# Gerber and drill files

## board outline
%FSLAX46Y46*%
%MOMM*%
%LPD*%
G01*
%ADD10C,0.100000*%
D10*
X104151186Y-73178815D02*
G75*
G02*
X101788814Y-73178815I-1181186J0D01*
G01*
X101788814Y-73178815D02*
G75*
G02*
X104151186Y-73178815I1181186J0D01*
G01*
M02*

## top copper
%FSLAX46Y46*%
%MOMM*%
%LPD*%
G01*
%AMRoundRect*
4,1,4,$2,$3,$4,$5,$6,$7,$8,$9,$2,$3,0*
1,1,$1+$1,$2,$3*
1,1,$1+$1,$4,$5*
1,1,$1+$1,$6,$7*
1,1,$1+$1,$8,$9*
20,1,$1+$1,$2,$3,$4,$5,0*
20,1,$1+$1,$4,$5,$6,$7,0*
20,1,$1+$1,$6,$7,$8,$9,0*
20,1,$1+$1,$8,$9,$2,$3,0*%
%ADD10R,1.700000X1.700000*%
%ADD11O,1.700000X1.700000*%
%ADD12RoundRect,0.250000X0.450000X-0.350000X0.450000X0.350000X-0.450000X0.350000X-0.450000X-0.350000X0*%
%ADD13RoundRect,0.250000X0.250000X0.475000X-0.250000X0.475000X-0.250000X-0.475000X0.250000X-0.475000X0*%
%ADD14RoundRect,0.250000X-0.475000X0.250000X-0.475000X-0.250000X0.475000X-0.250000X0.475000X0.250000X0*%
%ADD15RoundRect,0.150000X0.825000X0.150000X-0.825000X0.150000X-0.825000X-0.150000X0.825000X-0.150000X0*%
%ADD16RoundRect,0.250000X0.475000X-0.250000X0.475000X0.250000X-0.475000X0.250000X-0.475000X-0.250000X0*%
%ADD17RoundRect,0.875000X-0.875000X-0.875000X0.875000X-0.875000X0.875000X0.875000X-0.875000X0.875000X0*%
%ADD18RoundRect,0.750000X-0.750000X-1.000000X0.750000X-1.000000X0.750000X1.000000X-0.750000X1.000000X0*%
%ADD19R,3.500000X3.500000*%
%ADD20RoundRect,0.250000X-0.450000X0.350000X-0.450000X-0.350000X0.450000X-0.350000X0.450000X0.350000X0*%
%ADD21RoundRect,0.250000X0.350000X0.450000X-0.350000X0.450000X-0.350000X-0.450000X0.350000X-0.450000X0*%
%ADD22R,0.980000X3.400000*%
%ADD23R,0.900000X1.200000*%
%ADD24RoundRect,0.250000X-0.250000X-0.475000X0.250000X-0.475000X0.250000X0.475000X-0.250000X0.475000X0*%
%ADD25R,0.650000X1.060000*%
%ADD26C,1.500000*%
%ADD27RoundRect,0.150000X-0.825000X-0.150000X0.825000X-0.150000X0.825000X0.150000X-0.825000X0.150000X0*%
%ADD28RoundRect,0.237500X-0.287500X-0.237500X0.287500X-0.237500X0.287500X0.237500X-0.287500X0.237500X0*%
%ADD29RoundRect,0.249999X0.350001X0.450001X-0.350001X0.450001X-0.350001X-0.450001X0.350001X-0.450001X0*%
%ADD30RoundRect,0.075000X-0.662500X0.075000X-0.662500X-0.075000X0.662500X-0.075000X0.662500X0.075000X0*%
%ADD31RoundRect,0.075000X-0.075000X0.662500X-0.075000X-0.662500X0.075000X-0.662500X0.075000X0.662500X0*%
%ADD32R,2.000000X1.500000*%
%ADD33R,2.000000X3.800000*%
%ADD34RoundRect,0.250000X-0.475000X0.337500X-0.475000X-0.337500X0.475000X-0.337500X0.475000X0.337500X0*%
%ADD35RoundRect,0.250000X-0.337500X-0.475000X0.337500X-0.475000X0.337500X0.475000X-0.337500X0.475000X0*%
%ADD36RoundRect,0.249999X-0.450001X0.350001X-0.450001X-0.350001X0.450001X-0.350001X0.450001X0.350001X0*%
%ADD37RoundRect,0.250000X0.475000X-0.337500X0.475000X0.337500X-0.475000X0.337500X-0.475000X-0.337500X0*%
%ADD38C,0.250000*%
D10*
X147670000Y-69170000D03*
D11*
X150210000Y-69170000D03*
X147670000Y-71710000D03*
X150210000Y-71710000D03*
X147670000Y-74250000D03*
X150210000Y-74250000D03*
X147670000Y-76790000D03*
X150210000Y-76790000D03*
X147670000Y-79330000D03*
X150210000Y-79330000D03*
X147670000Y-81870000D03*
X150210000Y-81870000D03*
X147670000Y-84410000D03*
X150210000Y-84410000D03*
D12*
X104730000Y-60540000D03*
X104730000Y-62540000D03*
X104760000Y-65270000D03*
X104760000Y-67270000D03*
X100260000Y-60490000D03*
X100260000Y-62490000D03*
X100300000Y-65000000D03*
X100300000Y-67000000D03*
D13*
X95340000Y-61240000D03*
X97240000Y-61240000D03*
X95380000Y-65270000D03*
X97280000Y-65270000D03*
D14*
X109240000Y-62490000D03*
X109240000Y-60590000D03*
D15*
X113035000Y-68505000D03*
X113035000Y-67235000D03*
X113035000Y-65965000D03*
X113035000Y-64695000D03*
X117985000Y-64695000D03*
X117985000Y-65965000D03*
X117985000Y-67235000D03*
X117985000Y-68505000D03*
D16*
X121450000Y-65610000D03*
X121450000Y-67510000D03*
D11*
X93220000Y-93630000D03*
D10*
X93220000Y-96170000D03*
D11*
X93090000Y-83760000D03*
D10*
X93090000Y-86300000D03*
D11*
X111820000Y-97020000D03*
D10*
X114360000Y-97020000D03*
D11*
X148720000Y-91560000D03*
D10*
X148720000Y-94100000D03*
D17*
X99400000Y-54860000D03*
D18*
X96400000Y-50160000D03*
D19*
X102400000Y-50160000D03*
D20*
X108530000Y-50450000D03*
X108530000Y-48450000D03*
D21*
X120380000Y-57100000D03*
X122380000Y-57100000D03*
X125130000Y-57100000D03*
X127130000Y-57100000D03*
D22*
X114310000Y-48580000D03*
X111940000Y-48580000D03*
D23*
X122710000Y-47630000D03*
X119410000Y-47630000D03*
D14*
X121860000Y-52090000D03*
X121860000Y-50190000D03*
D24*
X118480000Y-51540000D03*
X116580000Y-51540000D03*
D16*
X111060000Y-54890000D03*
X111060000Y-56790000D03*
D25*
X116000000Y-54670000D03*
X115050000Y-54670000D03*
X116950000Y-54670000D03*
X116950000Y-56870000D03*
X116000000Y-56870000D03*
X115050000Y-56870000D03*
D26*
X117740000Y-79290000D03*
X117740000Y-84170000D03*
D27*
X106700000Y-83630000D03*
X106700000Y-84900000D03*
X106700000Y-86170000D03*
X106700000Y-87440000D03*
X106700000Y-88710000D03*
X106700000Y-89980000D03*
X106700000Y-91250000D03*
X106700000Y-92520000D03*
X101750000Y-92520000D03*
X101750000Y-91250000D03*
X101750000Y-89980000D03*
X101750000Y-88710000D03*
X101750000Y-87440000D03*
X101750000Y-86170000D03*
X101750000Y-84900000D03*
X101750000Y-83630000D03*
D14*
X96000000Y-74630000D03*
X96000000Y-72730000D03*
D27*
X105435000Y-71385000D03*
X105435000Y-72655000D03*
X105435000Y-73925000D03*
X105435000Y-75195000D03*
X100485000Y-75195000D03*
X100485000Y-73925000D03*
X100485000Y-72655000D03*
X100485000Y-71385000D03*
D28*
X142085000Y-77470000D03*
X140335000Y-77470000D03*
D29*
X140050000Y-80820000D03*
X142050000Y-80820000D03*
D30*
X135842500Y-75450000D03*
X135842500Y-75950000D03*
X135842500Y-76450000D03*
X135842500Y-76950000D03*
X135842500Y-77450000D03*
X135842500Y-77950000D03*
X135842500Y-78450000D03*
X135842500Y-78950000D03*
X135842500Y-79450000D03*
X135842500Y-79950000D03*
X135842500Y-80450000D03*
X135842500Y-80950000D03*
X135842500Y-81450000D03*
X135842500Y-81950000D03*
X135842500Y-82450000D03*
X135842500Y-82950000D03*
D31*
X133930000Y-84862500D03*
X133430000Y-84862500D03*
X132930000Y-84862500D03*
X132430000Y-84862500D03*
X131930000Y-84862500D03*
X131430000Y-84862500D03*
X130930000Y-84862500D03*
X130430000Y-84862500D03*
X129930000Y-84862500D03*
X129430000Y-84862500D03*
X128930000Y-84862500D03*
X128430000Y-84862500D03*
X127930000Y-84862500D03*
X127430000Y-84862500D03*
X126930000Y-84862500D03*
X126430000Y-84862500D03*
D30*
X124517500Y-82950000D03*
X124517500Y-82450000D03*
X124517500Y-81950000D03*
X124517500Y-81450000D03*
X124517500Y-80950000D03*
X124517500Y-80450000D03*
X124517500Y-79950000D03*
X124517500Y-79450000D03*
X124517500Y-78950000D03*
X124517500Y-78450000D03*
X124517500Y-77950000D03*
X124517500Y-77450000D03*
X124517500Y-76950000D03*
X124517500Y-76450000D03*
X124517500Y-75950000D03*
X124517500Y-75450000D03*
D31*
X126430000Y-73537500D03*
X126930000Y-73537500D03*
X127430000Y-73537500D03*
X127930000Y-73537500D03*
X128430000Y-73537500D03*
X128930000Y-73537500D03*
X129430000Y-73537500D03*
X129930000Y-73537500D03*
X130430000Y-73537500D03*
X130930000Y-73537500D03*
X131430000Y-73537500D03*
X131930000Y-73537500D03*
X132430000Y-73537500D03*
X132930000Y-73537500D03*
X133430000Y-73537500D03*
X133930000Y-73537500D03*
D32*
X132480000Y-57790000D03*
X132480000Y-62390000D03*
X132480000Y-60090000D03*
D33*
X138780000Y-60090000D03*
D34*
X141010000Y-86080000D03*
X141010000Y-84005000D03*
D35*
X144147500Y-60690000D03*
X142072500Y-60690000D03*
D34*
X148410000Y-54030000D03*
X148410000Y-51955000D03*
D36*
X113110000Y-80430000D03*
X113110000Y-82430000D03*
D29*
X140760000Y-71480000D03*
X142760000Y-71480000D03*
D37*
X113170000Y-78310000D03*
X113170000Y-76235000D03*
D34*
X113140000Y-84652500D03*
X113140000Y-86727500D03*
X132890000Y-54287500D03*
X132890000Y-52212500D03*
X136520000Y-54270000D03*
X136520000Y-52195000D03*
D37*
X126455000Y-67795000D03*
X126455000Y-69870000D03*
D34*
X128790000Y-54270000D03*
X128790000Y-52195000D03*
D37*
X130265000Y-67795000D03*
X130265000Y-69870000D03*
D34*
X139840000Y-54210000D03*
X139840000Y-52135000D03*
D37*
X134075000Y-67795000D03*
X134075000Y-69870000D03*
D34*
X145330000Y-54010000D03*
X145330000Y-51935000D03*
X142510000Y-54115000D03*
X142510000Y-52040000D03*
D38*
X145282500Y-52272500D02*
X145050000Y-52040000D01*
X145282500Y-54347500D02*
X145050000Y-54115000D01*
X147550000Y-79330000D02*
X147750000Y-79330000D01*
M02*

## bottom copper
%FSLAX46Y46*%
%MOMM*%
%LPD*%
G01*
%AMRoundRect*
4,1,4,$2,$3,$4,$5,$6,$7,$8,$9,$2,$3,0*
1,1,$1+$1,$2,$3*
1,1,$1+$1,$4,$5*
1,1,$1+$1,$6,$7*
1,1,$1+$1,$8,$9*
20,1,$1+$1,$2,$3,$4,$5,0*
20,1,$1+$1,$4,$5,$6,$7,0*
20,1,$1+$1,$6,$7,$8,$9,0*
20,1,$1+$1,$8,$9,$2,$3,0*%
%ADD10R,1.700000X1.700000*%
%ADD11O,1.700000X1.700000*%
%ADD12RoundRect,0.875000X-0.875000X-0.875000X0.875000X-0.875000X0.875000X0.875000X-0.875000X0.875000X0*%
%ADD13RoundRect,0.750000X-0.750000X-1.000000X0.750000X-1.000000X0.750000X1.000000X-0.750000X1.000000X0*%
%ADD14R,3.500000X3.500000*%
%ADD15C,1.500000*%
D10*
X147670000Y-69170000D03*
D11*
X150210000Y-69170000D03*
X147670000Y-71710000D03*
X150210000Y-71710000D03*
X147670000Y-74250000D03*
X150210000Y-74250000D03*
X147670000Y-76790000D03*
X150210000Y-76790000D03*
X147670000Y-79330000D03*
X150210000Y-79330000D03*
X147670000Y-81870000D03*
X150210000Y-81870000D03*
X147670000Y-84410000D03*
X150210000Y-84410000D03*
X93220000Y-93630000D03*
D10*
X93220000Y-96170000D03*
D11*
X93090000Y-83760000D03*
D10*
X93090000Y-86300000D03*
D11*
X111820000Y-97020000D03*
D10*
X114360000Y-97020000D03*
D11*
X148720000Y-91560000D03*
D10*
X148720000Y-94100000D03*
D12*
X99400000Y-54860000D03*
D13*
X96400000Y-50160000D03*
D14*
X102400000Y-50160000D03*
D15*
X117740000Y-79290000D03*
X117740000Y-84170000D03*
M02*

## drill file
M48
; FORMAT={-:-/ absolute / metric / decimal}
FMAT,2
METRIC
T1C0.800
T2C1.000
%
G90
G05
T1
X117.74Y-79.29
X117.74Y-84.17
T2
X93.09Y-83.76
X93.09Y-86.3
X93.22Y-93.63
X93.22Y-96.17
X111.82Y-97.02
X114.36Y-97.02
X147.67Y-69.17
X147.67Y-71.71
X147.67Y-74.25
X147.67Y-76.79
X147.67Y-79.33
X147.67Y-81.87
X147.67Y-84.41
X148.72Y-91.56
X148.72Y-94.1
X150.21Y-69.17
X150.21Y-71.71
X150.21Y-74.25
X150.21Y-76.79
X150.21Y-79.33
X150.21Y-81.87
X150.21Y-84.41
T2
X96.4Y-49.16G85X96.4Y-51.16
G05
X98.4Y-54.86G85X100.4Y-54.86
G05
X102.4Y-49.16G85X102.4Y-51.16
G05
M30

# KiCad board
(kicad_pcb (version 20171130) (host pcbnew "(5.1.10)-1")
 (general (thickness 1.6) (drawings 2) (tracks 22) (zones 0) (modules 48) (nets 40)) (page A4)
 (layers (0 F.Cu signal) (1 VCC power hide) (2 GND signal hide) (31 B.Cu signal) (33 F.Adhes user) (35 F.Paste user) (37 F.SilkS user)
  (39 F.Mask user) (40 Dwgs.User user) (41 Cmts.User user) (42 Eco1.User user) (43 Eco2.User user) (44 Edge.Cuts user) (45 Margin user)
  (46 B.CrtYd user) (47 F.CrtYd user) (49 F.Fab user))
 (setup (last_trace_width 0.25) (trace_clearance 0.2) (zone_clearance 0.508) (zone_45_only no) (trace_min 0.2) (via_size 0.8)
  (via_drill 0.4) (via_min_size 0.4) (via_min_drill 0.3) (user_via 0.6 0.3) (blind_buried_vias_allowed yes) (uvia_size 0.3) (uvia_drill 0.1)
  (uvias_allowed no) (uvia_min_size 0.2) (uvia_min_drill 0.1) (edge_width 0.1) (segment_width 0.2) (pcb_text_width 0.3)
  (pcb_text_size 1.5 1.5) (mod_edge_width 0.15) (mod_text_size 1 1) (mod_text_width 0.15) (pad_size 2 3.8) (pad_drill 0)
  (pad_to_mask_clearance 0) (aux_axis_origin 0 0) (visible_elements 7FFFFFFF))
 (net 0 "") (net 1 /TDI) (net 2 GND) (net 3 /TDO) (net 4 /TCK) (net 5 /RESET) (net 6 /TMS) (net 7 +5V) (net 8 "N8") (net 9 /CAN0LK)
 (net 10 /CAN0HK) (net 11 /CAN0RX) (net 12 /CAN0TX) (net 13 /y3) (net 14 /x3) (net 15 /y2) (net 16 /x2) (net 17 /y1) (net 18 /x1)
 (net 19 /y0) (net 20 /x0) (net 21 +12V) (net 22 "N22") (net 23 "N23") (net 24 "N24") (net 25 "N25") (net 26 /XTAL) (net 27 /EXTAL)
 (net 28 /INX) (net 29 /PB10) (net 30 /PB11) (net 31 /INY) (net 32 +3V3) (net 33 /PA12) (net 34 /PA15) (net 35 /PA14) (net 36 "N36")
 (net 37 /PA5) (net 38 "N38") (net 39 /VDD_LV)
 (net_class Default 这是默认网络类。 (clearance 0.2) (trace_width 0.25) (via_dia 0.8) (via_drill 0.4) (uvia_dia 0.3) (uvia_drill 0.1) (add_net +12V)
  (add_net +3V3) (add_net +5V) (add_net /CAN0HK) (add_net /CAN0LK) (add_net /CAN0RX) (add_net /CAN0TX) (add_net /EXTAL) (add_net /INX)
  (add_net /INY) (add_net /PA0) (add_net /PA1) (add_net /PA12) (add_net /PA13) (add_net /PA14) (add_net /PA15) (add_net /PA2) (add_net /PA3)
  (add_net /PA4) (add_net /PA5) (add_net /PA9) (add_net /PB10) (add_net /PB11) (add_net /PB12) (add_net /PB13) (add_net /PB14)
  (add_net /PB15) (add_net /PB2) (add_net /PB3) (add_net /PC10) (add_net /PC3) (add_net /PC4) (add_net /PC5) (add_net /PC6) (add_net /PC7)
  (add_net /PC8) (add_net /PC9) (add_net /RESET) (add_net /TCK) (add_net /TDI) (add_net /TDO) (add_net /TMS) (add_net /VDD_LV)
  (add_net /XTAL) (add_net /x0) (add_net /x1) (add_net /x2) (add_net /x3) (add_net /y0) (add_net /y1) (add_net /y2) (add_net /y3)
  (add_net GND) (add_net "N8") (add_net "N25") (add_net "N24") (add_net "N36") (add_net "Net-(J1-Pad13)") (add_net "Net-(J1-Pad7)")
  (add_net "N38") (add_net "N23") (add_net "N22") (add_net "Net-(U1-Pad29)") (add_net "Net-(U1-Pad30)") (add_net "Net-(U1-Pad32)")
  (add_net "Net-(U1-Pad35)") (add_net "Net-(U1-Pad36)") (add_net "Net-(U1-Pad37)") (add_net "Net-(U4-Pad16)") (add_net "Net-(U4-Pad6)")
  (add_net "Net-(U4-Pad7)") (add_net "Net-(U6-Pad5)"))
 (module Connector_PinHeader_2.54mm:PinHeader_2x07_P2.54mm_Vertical (layer F.Cu) (at 147.67 69.17)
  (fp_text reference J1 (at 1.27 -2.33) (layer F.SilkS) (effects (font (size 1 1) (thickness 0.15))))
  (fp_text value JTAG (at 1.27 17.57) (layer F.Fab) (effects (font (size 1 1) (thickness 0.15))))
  (pad 1 thru_hole rect (at 0 0) (size 1.7 1.7) (drill 1) (layers *.Cu *.Mask) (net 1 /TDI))
  (pad 2 thru_hole oval (at 2.54 0) (size 1.7 1.7) (drill 1) (layers *.Cu *.Mask) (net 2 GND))
  (pad 3 thru_hole oval (at 0 2.54) (size 1.7 1.7) (drill 1) (layers *.Cu *.Mask) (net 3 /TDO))
  (pad 4 thru_hole oval (at 2.54 2.54) (size 1.7 1.7) (drill 1) (layers *.Cu *.Mask) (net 2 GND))
  (pad 5 thru_hole oval (at 0 5.08) (size 1.7 1.7) (drill 1) (layers *.Cu *.Mask) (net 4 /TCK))
  (pad 6 thru_hole oval (at 2.54 5.08) (size 1.7 1.7) (drill 1) (layers *.Cu *.Mask) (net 2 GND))
  (pad 7 thru_hole oval (at 0 7.62) (size 1.7 1.7) (drill 1) (layers *.Cu *.Mask))
  (pad 8 thru_hole oval (at 2.54 7.62) (size 1.7 1.7) (drill 1) (layers *.Cu *.Mask) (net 2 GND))
  (pad 9 thru_hole oval (at 0 10.16) (size 1.7 1.7) (drill 1) (layers *.Cu *.Mask) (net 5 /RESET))
  (pad 10 thru_hole oval (at 2.54 10.16) (size 1.7 1.7) (drill 1) (layers *.Cu *.Mask) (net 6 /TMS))
  (pad 11 thru_hole oval (at 0 12.7) (size 1.7 1.7) (drill 1) (layers *.Cu *.Mask) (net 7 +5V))
  (pad 12 thru_hole oval (at 2.54 12.7) (size 1.7 1.7) (drill 1) (layers *.Cu *.Mask) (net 2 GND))
  (pad 13 thru_hole oval (at 0 15.24) (size 1.7 1.7) (drill 1) (layers *.Cu *.Mask))
  (pad 14 thru_hole oval (at 2.54 15.24) (size 1.7 1.7) (drill 1) (layers *.Cu *.Mask) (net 2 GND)))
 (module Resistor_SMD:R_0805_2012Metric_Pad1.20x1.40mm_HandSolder (layer F.Cu) (at 104.73 61.54 90)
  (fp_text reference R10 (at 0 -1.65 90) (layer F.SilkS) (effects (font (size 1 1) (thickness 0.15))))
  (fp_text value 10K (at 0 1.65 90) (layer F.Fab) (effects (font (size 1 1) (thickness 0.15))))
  (pad 2 smd roundrect (at 1 0 90) (size 1.2 1.4) (layers F.Cu F.Paste F.Mask) (roundrect_rratio 0.208333) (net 2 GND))
  (pad 1 smd roundrect (at -1 0 90) (size 1.2 1.4) (layers F.Cu F.Paste F.Mask) (roundrect_rratio 0.208333) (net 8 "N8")))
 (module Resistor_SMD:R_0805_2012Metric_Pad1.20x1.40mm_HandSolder (layer F.Cu) (at 104.76 66.27 90)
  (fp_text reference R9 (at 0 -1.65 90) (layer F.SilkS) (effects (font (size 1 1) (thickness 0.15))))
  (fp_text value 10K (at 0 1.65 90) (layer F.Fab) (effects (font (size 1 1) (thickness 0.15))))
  (pad 2 smd roundrect (at 1 0 90) (size 1.2 1.4) (layers F.Cu F.Paste F.Mask) (roundrect_rratio 0.208333) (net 8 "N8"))
  (pad 1 smd roundrect (at -1 0 90) (size 1.2 1.4) (layers F.Cu F.Paste F.Mask) (roundrect_rratio 0.208333) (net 7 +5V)))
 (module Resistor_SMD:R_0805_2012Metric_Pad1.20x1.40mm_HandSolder (layer F.Cu) (at 100.26 61.49 90)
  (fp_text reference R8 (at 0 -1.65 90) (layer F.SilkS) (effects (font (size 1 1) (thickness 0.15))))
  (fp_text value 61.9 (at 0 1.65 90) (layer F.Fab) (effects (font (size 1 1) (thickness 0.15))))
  (pad 2 smd roundrect (at 1 0 90) (size 1.2 1.4) (layers F.Cu F.Paste F.Mask) (roundrect_rratio 0.208333) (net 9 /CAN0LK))
  (pad 1 smd roundrect (at -1 0 90) (size 1.2 1.4) (layers F.Cu F.Paste F.Mask) (roundrect_rratio 0.208333) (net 8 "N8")))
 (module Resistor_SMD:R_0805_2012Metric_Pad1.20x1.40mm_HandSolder (layer F.Cu) (at 100.3 66 90)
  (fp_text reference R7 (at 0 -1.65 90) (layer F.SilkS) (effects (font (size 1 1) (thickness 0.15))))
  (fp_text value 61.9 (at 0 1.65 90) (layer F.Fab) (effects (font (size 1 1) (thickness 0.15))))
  (pad 2 smd roundrect (at 1 0 90) (size 1.2 1.4) (layers F.Cu F.Paste F.Mask) (roundrect_rratio 0.208333) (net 8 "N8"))
  (pad 1 smd roundrect (at -1 0 90) (size 1.2 1.4) (layers F.Cu F.Paste F.Mask) (roundrect_rratio 0.208333) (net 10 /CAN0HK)))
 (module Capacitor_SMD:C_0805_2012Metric (layer F.Cu) (at 96.29 61.24 180)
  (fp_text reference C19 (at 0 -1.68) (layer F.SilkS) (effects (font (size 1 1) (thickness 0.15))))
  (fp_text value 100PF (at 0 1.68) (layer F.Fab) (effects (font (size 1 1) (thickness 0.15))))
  (pad 2 smd roundrect (at 0.95 0 180) (size 1 1.45) (layers F.Cu F.Paste F.Mask) (roundrect_rratio 0.25) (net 2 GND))
  (pad 1 smd roundrect (at -0.95 0 180) (size 1 1.45) (layers F.Cu F.Paste F.Mask) (roundrect_rratio 0.25) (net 9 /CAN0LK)))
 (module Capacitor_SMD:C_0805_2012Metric (layer F.Cu) (at 96.33 65.27 180)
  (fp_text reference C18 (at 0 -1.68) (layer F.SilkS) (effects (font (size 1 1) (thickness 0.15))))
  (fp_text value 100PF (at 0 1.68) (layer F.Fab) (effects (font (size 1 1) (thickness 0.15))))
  (pad 2 smd roundrect (at 0.95 0 180) (size 1 1.45) (layers F.Cu F.Paste F.Mask) (roundrect_rratio 0.25) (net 2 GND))
  (pad 1 smd roundrect (at -0.95 0 180) (size 1 1.45) (layers F.Cu F.Paste F.Mask) (roundrect_rratio 0.25) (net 10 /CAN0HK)))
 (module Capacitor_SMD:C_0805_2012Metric (layer F.Cu) (at 109.24 61.54 270)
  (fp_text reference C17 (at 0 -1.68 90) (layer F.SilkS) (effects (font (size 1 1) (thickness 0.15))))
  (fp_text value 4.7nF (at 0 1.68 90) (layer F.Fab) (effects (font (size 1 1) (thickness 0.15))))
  (pad 2 smd roundrect (at 0.95 0 270) (size 1 1.45) (layers F.Cu F.Paste F.Mask) (roundrect_rratio 0.25) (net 8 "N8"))
  (pad 1 smd roundrect (at -0.95 0 270) (size 1 1.45) (layers F.Cu F.Paste F.Mask) (roundrect_rratio 0.25) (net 2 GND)))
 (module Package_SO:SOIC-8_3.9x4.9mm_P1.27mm (layer F.Cu) (at 115.51 66.6 180)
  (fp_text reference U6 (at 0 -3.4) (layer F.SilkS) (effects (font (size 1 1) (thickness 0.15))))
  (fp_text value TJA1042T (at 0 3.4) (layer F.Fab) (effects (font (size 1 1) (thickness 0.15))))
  (pad 8 smd roundrect (at 2.475 -1.905 180) (size 1.95 0.6) (layers F.Cu F.Paste F.Mask) (roundrect_rratio 0.25) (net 2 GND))
  (pad 7 smd roundrect (at 2.475 -0.635 180) (size 1.95 0.6) (layers F.Cu F.Paste F.Mask) (roundrect_rratio 0.25) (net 10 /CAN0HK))
  (pad 6 smd roundrect (at 2.475 0.635 180) (size 1.95 0.6) (layers F.Cu F.Paste F.Mask) (roundrect_rratio 0.25) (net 9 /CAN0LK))
  (pad 5 smd roundrect (at 2.475 1.905 180) (size 1.95 0.6) (layers F.Cu F.Paste F.Mask) (roundrect_rratio 0.25))
  (pad 4 smd roundrect (at -2.475 1.905 180) (size 1.95 0.6) (layers F.Cu F.Paste F.Mask) (roundrect_rratio 0.25) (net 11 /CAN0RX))
  (pad 3 smd roundrect (at -2.475 0.635 180) (size 1.95 0.6) (layers F.Cu F.Paste F.Mask) (roundrect_rratio 0.25) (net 7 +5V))
  (pad 2 smd roundrect (at -2.475 -0.635 180) (size 1.95 0.6) (layers F.Cu F.Paste F.Mask) (roundrect_rratio 0.25) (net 2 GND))
  (pad 1 smd roundrect (at -2.475 -1.905 180) (size 1.95 0.6) (layers F.Cu F.Paste F.Mask) (roundrect_rratio 0.25) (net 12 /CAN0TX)))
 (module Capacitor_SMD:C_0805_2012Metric (layer F.Cu) (at 121.45 66.56 90)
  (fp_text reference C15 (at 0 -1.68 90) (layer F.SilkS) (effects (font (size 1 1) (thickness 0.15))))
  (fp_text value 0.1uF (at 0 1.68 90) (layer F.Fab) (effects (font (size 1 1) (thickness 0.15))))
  (pad 2 smd roundrect (at 0.95 0 90) (size 1 1.45) (layers F.Cu F.Paste F.Mask) (roundrect_rratio 0.25) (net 7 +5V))
  (pad 1 smd roundrect (at -0.95 0 90) (size 1 1.45) (layers F.Cu F.Paste F.Mask) (roundrect_rratio 0.25) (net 2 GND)))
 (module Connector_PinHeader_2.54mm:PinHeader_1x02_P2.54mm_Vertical (layer F.Cu) (at 93.22 96.17 180)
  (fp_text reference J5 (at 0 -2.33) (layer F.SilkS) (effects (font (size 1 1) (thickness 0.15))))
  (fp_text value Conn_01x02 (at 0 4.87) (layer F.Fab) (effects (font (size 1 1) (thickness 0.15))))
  (pad 2 thru_hole oval (at 0 2.54 180) (size 1.7 1.7) (drill 1) (layers *.Cu *.Mask) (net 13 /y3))
  (pad 1 thru_hole rect (at 0 0 180) (size 1.7 1.7) (drill 1) (layers *.Cu *.Mask) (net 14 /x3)))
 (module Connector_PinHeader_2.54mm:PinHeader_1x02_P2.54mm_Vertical (layer F.Cu) (at 93.09 86.3 180)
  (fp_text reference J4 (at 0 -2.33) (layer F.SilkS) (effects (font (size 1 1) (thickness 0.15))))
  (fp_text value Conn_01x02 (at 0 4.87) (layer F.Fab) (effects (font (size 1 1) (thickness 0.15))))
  (pad 2 thru_hole oval (at 0 2.54 180) (size 1.7 1.7) (drill 1) (layers *.Cu *.Mask) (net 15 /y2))
  (pad 1 thru_hole rect (at 0 0 180) (size 1.7 1.7) (drill 1) (layers *.Cu *.Mask) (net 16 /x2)))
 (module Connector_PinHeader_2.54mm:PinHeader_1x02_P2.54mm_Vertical (layer F.Cu) (at 114.36 97.02 270)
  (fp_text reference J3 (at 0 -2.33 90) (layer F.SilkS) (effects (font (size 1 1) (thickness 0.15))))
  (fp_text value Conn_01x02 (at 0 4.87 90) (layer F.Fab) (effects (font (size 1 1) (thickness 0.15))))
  (pad 2 thru_hole oval (at 0 2.54 270) (size 1.7 1.7) (drill 1) (layers *.Cu *.Mask) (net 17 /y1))
  (pad 1 thru_hole rect (at 0 0 270) (size 1.7 1.7) (drill 1) (layers *.Cu *.Mask) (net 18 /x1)))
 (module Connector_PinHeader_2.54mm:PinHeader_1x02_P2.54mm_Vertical (layer F.Cu) (at 148.72 94.1 180)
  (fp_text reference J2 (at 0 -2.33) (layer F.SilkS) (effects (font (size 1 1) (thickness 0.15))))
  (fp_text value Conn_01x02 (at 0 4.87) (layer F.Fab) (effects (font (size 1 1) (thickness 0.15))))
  (pad 2 thru_hole oval (at 0 2.54 180) (size 1.7 1.7) (drill 1) (layers *.Cu *.Mask) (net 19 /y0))
  (pad 1 thru_hole rect (at 0 0 180) (size 1.7 1.7) (drill 1) (layers *.Cu *.Mask) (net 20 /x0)))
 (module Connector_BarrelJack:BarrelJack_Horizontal (layer F.Cu) (at 102.4 50.16)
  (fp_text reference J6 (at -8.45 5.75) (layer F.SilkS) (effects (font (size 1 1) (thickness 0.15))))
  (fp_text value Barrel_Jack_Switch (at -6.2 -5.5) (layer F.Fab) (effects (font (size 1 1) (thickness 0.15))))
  (pad 3 thru_hole roundrect (at -3 4.7) (size 3.5 3.5) (drill oval 3 1) (layers *.Cu *.Mask) (roundrect_rratio 0.25) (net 2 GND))
  (pad 2 thru_hole roundrect (at -6 0) (size 3 3.5) (drill oval 1 3) (layers *.Cu *.Mask) (roundrect_rratio 0.25) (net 2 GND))
  (pad 1 thru_hole rect (at 0 0) (size 3.5 3.5) (drill oval 1 3) (layers *.Cu *.Mask) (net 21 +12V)))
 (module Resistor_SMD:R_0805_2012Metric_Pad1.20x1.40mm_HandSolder (layer F.Cu) (at 108.53 49.45 270)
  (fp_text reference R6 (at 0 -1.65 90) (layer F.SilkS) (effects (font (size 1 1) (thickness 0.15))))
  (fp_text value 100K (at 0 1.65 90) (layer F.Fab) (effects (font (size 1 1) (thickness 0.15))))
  (pad 2 smd roundrect (at 1 0 270) (size 1.2 1.4) (layers F.Cu F.Paste F.Mask) (roundrect_rratio 0.208333) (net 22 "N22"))
  (pad 1 smd roundrect (at -1 0 270) (size 1.2 1.4) (layers F.Cu F.Paste F.Mask) (roundrect_rratio 0.208333) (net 21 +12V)))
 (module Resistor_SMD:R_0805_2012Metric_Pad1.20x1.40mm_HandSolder (layer F.Cu) (at 121.38 57.1 180)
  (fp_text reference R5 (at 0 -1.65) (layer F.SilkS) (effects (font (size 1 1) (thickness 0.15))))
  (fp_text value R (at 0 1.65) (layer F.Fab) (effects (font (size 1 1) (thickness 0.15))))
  (pad 2 smd roundrect (at 1 0 180) (size 1.2 1.4) (layers F.Cu F.Paste F.Mask) (roundrect_rratio 0.208333) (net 2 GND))
  (pad 1 smd roundrect (at -1 0 180) (size 1.2 1.4) (layers F.Cu F.Paste F.Mask) (roundrect_rratio 0.208333) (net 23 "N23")))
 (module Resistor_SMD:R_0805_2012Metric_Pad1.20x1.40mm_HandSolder (layer F.Cu) (at 126.13 57.1 180)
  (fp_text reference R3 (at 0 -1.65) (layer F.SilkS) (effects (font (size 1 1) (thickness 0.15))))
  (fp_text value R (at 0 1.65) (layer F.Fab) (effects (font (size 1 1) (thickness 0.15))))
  (pad 2 smd roundrect (at 1 0 180) (size 1.2 1.4) (layers F.Cu F.Paste F.Mask) (roundrect_rratio 0.208333) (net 23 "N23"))
  (pad 1 smd roundrect (at -1 0 180) (size 1.2 1.4) (layers F.Cu F.Paste F.Mask) (roundrect_rratio 0.208333) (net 7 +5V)))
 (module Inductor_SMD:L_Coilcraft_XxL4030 (layer F.Cu) (at 113.125 48.58)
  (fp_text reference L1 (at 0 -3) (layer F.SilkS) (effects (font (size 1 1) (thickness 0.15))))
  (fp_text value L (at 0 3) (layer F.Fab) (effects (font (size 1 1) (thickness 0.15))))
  (pad 2 smd rect (at 1.185 0) (size 0.98 3.4) (layers F.Cu F.Paste F.Mask) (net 7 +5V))
  (pad 1 smd rect (at -1.185 0) (size 0.98 3.4) (layers F.Cu F.Paste F.Mask) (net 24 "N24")))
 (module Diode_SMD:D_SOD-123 (layer F.Cu) (at 121.06 47.63)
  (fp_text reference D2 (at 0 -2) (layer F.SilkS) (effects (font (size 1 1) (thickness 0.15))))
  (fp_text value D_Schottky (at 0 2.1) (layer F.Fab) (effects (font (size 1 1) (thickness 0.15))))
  (pad 2 smd rect (at 1.65 0) (size 0.9 1.2) (layers F.Cu F.Paste F.Mask) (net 2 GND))
  (pad 1 smd rect (at -1.65 0) (size 0.9 1.2) (layers F.Cu F.Paste F.Mask) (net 24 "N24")))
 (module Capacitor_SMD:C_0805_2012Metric (layer F.Cu) (at 121.86 51.14 270)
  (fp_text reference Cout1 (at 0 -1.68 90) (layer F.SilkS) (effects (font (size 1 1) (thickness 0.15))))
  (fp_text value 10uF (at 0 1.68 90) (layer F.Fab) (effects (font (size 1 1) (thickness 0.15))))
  (pad 2 smd roundrect (at 0.95 0 270) (size 1 1.45) (layers F.Cu F.Paste F.Mask) (roundrect_rratio 0.25) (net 2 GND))
  (pad 1 smd roundrect (at -0.95 0 270) (size 1 1.45) (layers F.Cu F.Paste F.Mask) (roundrect_rratio 0.25) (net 7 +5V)))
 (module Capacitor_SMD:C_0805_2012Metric (layer F.Cu) (at 117.53 51.54)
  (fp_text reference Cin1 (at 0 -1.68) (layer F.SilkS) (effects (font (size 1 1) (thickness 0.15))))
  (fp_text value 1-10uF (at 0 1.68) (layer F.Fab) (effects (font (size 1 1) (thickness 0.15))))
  (pad 2 smd roundrect (at 0.95 0) (size 1 1.45) (layers F.Cu F.Paste F.Mask) (roundrect_rratio 0.25) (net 2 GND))
  (pad 1 smd roundrect (at -0.95 0) (size 1 1.45) (layers F.Cu F.Paste F.Mask) (roundrect_rratio 0.25) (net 21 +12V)))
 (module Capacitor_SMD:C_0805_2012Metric (layer F.Cu) (at 111.06 55.84 90)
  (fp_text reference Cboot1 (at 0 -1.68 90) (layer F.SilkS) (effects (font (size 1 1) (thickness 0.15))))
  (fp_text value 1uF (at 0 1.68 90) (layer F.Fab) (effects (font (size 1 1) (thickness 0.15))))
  (pad 2 smd roundrect (at 0.95 0 90) (size 1 1.45) (layers F.Cu F.Paste F.Mask) (roundrect_rratio 0.25) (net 24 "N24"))
  (pad 1 smd roundrect (at -0.95 0 90) (size 1 1.45) (layers F.Cu F.Paste F.Mask) (roundrect_rratio 0.25) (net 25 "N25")))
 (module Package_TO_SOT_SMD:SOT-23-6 (layer F.Cu) (at 116 55.77 90)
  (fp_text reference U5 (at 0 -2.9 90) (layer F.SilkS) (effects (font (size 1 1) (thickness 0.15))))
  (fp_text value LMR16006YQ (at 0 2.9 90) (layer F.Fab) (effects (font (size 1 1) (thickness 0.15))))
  (pad 5 smd rect (at 1.1 0 90) (size 1.06 0.65) (layers F.Cu F.Paste F.Mask) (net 21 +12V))
  (pad 6 smd rect (at 1.1 -0.95 90) (size 1.06 0.65) (layers F.Cu F.Paste F.Mask) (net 24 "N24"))
  (pad 4 smd rect (at 1.1 0.95 90) (size 1.06 0.65) (layers F.Cu F.Paste F.Mask) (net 22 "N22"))
  (pad 3 smd rect (at -1.1 0.95 90) (size 1.06 0.65) (layers F.Cu F.Paste F.Mask) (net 23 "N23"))
  (pad 2 smd rect (at -1.1 0 90) (size 1.06 0.65) (layers F.Cu F.Paste F.Mask) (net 2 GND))
  (pad 1 smd rect (at -1.1 -0.95 90) (size 1.06 0.65) (layers F.Cu F.Paste F.Mask) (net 25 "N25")))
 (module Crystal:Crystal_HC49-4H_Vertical (layer F.Cu) (at 117.74 84.17 90)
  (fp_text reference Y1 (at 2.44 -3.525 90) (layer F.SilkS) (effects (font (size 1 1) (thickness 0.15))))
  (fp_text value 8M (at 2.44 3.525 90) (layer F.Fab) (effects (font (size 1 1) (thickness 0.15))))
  (pad 2 thru_hole circle (at 4.88 0 90) (size 1.5 1.5) (drill 0.8) (layers *.Cu *.Mask) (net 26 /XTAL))
  (pad 1 thru_hole circle (at 0 0 90) (size 1.5 1.5) (drill 0.8) (layers *.Cu *.Mask) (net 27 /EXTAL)))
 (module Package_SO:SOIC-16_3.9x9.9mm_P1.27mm (layer F.Cu) (at 104.225 88.075)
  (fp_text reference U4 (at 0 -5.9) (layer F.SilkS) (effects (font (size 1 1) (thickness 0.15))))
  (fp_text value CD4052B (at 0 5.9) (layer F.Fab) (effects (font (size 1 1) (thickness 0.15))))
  (pad 16 smd roundrect (at 2.475 -4.445) (size 1.95 0.6) (layers F.Cu F.Paste F.Mask) (roundrect_rratio 0.25))
  (pad 15 smd roundrect (at 2.475 -3.175) (size 1.95 0.6) (layers F.Cu F.Paste F.Mask) (roundrect_rratio 0.25) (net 16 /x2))
  (pad 14 smd roundrect (at 2.475 -1.905) (size 1.95 0.6) (layers F.Cu F.Paste F.Mask) (roundrect_rratio 0.25) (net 18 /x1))
  (pad 13 smd roundrect (at 2.475 -0.635) (size 1.95 0.6) (layers F.Cu F.Paste F.Mask) (roundrect_rratio 0.25) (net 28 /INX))
  (pad 12 smd roundrect (at 2.475 0.635) (size 1.95 0.6) (layers F.Cu F.Paste F.Mask) (roundrect_rratio 0.25) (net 20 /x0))
  (pad 11 smd roundrect (at 2.475 1.905) (size 1.95 0.6) (layers F.Cu F.Paste F.Mask) (roundrect_rratio 0.25) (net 14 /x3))
  (pad 10 smd roundrect (at 2.475 3.175) (size 1.95 0.6) (layers F.Cu F.Paste F.Mask) (roundrect_rratio 0.25) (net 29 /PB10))
  (pad 9 smd roundrect (at 2.475 4.445) (size 1.95 0.6) (layers F.Cu F.Paste F.Mask) (roundrect_rratio 0.25) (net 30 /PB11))
  (pad 8 smd roundrect (at -2.475 4.445) (size 1.95 0.6) (layers F.Cu F.Paste F.Mask) (roundrect_rratio 0.25) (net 2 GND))
  (pad 7 smd roundrect (at -2.475 3.175) (size 1.95 0.6) (layers F.Cu F.Paste F.Mask) (roundrect_rratio 0.25))
  (pad 6 smd roundrect (at -2.475 1.905) (size 1.95 0.6) (layers F.Cu F.Paste F.Mask) (roundrect_rratio 0.25))
  (pad 5 smd roundrect (at -2.475 0.635) (size 1.95 0.6) (layers F.Cu F.Paste F.Mask) (roundrect_rratio 0.25) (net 17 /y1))
  (pad 4 smd roundrect (at -2.475 -0.635) (size 1.95 0.6) (layers F.Cu F.Paste F.Mask) (roundrect_rratio 0.25) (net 13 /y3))
  (pad 3 smd roundrect (at -2.475 -1.905) (size 1.95 0.6) (layers F.Cu F.Paste F.Mask) (roundrect_rratio 0.25) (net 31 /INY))
  (pad 2 smd roundrect (at -2.475 -3.175) (size 1.95 0.6) (layers F.Cu F.Paste F.Mask) (roundrect_rratio 0.25) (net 15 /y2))
  (pad 1 smd roundrect (at -2.475 -4.445) (size 1.95 0.6) (layers F.Cu F.Paste F.Mask) (roundrect_rratio 0.25) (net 19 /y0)))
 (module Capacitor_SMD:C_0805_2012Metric (layer F.Cu) (at 96 73.68 270)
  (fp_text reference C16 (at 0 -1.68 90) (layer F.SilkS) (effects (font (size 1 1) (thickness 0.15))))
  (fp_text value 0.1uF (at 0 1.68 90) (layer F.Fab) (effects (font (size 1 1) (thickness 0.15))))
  (pad 2 smd roundrect (at 0.95 0 270) (size 1 1.45) (layers F.Cu F.Paste F.Mask) (roundrect_rratio 0.25) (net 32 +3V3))
  (pad 1 smd roundrect (at -0.95 0 270) (size 1 1.45) (layers F.Cu F.Paste F.Mask) (roundrect_rratio 0.25) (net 2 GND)))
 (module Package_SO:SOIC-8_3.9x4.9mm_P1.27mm (layer F.Cu) (at 102.96 73.29)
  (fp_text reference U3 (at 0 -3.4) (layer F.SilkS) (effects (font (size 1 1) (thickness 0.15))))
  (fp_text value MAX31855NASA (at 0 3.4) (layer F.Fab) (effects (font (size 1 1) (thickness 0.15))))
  (pad 8 smd roundrect (at 2.475 -1.905) (size 1.95 0.6) (layers F.Cu F.Paste F.Mask) (roundrect_rratio 0.25))
  (pad 7 smd roundrect (at 2.475 -0.635) (size 1.95 0.6) (layers F.Cu F.Paste F.Mask) (roundrect_rratio 0.25) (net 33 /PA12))
  (pad 6 smd roundrect (at 2.475 0.635) (size 1.95 0.6) (layers F.Cu F.Paste F.Mask) (roundrect_rratio 0.25) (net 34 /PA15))
  (pad 5 smd roundrect (at 2.475 1.905) (size 1.95 0.6) (layers F.Cu F.Paste F.Mask) (roundrect_rratio 0.25) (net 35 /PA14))
  (pad 4 smd roundrect (at -2.475 1.905) (size 1.95 0.6) (layers F.Cu F.Paste F.Mask) (roundrect_rratio 0.25) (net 32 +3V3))
  (pad 3 smd roundrect (at -2.475 0.635) (size 1.95 0.6) (layers F.Cu F.Paste F.Mask) (roundrect_rratio 0.25) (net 28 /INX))
  (pad 2 smd roundrect (at -2.475 -0.635) (size 1.95 0.6) (layers F.Cu F.Paste F.Mask) (roundrect_rratio 0.25) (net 31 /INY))
  (pad 1 smd roundrect (at -2.475 -1.905) (size 1.95 0.6) (layers F.Cu F.Paste F.Mask) (roundrect_rratio 0.25) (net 2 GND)))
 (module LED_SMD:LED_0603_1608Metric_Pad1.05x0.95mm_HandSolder (layer F.Cu) (at 141.21 77.47)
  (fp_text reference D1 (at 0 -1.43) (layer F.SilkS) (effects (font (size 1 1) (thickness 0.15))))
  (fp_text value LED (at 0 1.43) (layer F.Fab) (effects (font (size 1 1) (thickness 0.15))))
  (pad 2 smd roundrect (at 0.875 0) (size 1.05 0.95) (layers F.Cu F.Paste F.Mask) (roundrect_rratio 0.25) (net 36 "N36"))
  (pad 1 smd roundrect (at -0.875 0) (size 1.05 0.95) (layers F.Cu F.Paste F.Mask) (roundrect_rratio 0.25) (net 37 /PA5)))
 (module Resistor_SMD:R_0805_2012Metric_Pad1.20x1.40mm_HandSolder (layer F.Cu) (at 141.05 80.82 180)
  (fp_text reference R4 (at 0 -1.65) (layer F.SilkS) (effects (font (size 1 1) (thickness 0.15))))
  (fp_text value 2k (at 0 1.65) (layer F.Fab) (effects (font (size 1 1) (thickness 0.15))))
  (pad 2 smd roundrect (at 1 0 180) (size 1.2 1.4) (layers F.Cu F.Paste F.Mask) (roundrect_rratio 0.2083325) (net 7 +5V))
  (pad 1 smd roundrect (at -1 0 180) (size 1.2 1.4) (layers F.Cu F.Paste F.Mask) (roundrect_rratio 0.2083325) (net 36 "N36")))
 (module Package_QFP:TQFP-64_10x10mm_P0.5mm (layer F.Cu) (at 130.18 79.2 270)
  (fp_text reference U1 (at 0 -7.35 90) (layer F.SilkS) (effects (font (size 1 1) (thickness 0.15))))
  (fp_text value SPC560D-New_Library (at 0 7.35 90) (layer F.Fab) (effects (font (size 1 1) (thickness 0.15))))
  (pad 64 smd roundrect (at -3.75 -5.6625 270) (size 0.3 1.475) (layers F.Cu F.Paste F.Mask) (roundrect_rratio 0.25))
  (pad 63 smd roundrect (at -3.25 -5.6625 270) (size 0.3 1.475) (layers F.Cu F.Paste F.Mask) (roundrect_rratio 0.25))
  (pad 62 smd roundrect (at -2.75 -5.6625 270) (size 0.3 1.475) (layers F.Cu F.Paste F.Mask) (roundrect_rratio 0.25))
  (pad 61 smd roundrect (at -2.25 -5.6625 270) (size 0.3 1.475) (layers F.Cu F.Paste F.Mask) (roundrect_rratio 0.25))
  (pad 60 smd roundrect (at -1.75 -5.6625 270) (size 0.3 1.475) (layers F.Cu F.Paste F.Mask) (roundrect_rratio 0.25) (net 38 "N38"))
  (pad 59 smd roundrect (at -1.25 -5.6625 270) (size 0.3 1.475) (layers F.Cu F.Paste F.Mask) (roundrect_rratio 0.25) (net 1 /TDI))
  (pad 58 smd roundrect (at -0.75 -5.6625 270) (size 0.3 1.475) (layers F.Cu F.Paste F.Mask) (roundrect_rratio 0.25) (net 2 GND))
  (pad 57 smd roundrect (at -0.25 -5.6625 270) (size 0.3 1.475) (layers F.Cu F.Paste F.Mask) (roundrect_rratio 0.25) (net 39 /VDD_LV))
  (pad 56 smd roundrect (at 0.25 -5.6625 270) (size 0.3 1.475) (layers F.Cu F.Paste F.Mask) (roundrect_rratio 0.25) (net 7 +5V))
  (pad 55 smd roundrect (at 0.75 -5.6625 270) (size 0.3 1.475) (layers F.Cu F.Paste F.Mask) (roundrect_rratio 0.25) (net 2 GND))
  (pad 54 smd roundrect (at 1.25 -5.6625 270) (size 0.3 1.475) (layers F.Cu F.Paste F.Mask) (roundrect_rratio 0.25) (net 3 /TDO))
  (pad 53 smd roundrect (at 1.75 -5.6625 270) (size 0.3 1.475) (layers F.Cu F.Paste F.Mask) (roundrect_rratio 0.25) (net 6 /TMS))
  (pad 52 smd roundrect (at 2.25 -5.6625 270) (size 0.3 1.475) (layers F.Cu F.Paste F.Mask) (roundrect_rratio 0.25))
  (pad 51 smd roundrect (at 2.75 -5.6625 270) (size 0.3 1.475) (layers F.Cu F.Paste F.Mask) (roundrect_rratio 0.25) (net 37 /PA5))
  (pad 50 smd roundrect (at 3.25 -5.6625 270) (size 0.3 1.475) (layers F.Cu F.Paste F.Mask) (roundrect_rratio 0.25))
  (pad 49 smd roundrect (at 3.75 -5.6625 270) (size 0.3 1.475) (layers F.Cu F.Paste F.Mask) (roundrect_rratio 0.25))
  (pad 48 smd roundrect (at 5.6625 -3.75 270) (size 1.475 0.3) (layers F.Cu F.Paste F.Mask) (roundrect_rratio 0.25))
  (pad 47 smd roundrect (at 5.6625 -3.25 270) (size 1.475 0.3) (layers F.Cu F.Paste F.Mask) (roundrect_rratio 0.25))
  (pad 46 smd roundrect (at 5.6625 -2.75 270) (size 1.475 0.3) (layers F.Cu F.Paste F.Mask) (roundrect_rratio 0.25))
  (pad 45 smd roundrect (at 5.6625 -2.25 270) (size 1.475 0.3) (layers F.Cu F.Paste F.Mask) (roundrect_rratio 0.25))
  (pad 44 smd roundrect (at 5.6625 -1.75 270) (size 1.475 0.3) (layers F.Cu F.Paste F.Mask) (roundrect_rratio 0.25))
  (pad 43 smd roundrect (at 5.6625 -1.25 270) (size 1.475 0.3) (layers F.Cu F.Paste F.Mask) (roundrect_rratio 0.25))
  (pad 42 smd roundrect (at 5.6625 -0.75 270) (size 1.475 0.3) (layers F.Cu F.Paste F.Mask) (roundrect_rratio 0.25))
  (pad 41 smd roundrect (at 5.6625 -0.25 270) (size 1.475 0.3) (layers F.Cu F.Paste F.Mask) (roundrect_rratio 0.25))
  (pad 40 smd roundrect (at 5.6625 0.25 270) (size 1.475 0.3) (layers F.Cu F.Paste F.Mask) (roundrect_rratio 0.25))
  (pad 39 smd roundrect (at 5.6625 0.75 270) (size 1.475 0.3) (layers F.Cu F.Paste F.Mask) (roundrect_rratio 0.25))
  (pad 38 smd roundrect (at 5.6625 1.25 270) (size 1.475 0.3) (layers F.Cu F.Paste F.Mask) (roundrect_rratio 0.25) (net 30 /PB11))
  (pad 37 smd roundrect (at 5.6625 1.75 270) (size 1.475 0.3) (layers F.Cu F.Paste F.Mask) (roundrect_rratio 0.25))
  (pad 36 smd roundrect (at 5.6625 2.25 270) (size 1.475 0.3) (layers F.Cu F.Paste F.Mask) (roundrect_rratio 0.25))
  (pad 35 smd roundrect (at 5.6625 2.75 270) (size 1.475 0.3) (layers F.Cu F.Paste F.Mask) (roundrect_rratio 0.25))
  (pad 34 smd roundrect (at 5.6625 3.25 270) (size 1.475 0.3) (layers F.Cu F.Paste F.Mask) (roundrect_rratio 0.25) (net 7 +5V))
  (pad 33 smd roundrect (at 5.6625 3.75 270) (size 1.475 0.3) (layers F.Cu F.Paste F.Mask) (roundrect_rratio 0.25) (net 2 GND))
  (pad 32 smd roundrect (at 3.75 5.6625 270) (size 0.3 1.475) (layers F.Cu F.Paste F.Mask) (roundrect_rratio 0.25))
  (pad 31 smd roundrect (at 3.25 5.6625 270) (size 0.3 1.475) (layers F.Cu F.Paste F.Mask) (roundrect_rratio 0.25) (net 29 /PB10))
  (pad 30 smd roundrect (at 2.75 5.6625 270) (size 0.3 1.475) (layers F.Cu F.Paste F.Mask) (roundrect_rratio 0.25))
  (pad 29 smd roundrect (at 2.25 5.6625 270) (size 0.3 1.475) (layers F.Cu F.Paste F.Mask) (roundrect_rratio 0.25))
  (pad 28 smd roundrect (at 1.75 5.6625 270) (size 0.3 1.475) (layers F.Cu F.Paste F.Mask) (roundrect_rratio 0.25) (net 7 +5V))
  (pad 27 smd roundrect (at 1.25 5.6625 270) (size 0.3 1.475) (layers F.Cu F.Paste F.Mask) (roundrect_rratio 0.25) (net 27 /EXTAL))
  (pad 26 smd roundrect (at 0.75 5.6625 270) (size 0.3 1.475) (layers F.Cu F.Paste F.Mask) (roundrect_rratio 0.25) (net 2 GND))
  (pad 25 smd roundrect (at 0.25 5.6625 270) (size 0.3 1.475) (layers F.Cu F.Paste F.Mask) (roundrect_rratio 0.25) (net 26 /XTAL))
  (pad 24 smd roundrect (at -0.25 5.6625 270) (size 0.3 1.475) (layers F.Cu F.Paste F.Mask) (roundrect_rratio 0.25) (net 2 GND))
  (pad 23 smd roundrect (at -0.75 5.6625 270) (size 0.3 1.475) (layers F.Cu F.Paste F.Mask) (roundrect_rratio 0.25) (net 39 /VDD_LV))
  (pad 22 smd roundrect (at -1.25 5.6625 270) (size 0.3 1.475) (layers F.Cu F.Paste F.Mask) (roundrect_rratio 0.25) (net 33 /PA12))
  (pad 21 smd roundrect (at -1.75 5.6625 270) (size 0.3 1.475) (layers F.Cu F.Paste F.Mask) (roundrect_rratio 0.25))
  (pad 20 smd roundrect (at -2.25 5.6625 270) (size 0.3 1.475) (layers F.Cu F.Paste F.Mask) (roundrect_rratio 0.25))
  (pad 19 smd roundrect (at -2.75 5.6625 270) (size 0.3 1.475) (layers F.Cu F.Paste F.Mask) (roundrect_rratio 0.25) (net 35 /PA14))
  (pad 18 smd roundrect (at -3.25 5.6625 270) (size 0.3 1.475) (layers F.Cu F.Paste F.Mask) (roundrect_rratio 0.25) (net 34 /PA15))
  (pad 17 smd roundrect (at -3.75 5.6625 270) (size 0.3 1.475) (layers F.Cu F.Paste F.Mask) (roundrect_rratio 0.25))
  (pad 16 smd roundrect (at -5.6625 3.75 270) (size 1.475 0.3) (layers F.Cu F.Paste F.Mask) (roundrect_rratio 0.25))
  (pad 15 smd roundrect (at -5.6625 3.25 270) (size 1.475 0.3) (layers F.Cu F.Paste F.Mask) (roundrect_rratio 0.25) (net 11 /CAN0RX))
  (pad 14 smd roundrect (at -5.6625 2.75 270) (size 1.475 0.3) (layers F.Cu F.Paste F.Mask) (roundrect_rratio 0.25) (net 12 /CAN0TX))
  (pad 13 smd roundrect (at -5.6625 2.25 270) (size 1.475 0.3) (layers F.Cu F.Paste F.Mask) (roundrect_rratio 0.25))
  (pad 12 smd roundrect (at -5.6625 1.75 270) (size 1.475 0.3) (layers F.Cu F.Paste F.Mask) (roundrect_rratio 0.25) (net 7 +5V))
  (pad 11 smd roundrect (at -5.6625 1.25 270) (size 1.475 0.3) (layers F.Cu F.Paste F.Mask) (roundrect_rratio 0.25) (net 39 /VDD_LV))
  (pad 10 smd roundrect (at -5.6625 0.75 270) (size 1.475 0.3) (layers F.Cu F.Paste F.Mask) (roundrect_rratio 0.25) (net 2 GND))
  (pad 9 smd roundrect (at -5.6625 0.25 270) (size 1.475 0.3) (layers F.Cu F.Paste F.Mask) (roundrect_rratio 0.25) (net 5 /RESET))
  (pad 8 smd roundrect (at -5.6625 -0.25 270) (size 1.475 0.3) (layers F.Cu F.Paste F.Mask) (roundrect_rratio 0.25) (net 2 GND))
  (pad 7 smd roundrect (at -5.6625 -0.75 270) (size 1.475 0.3) (layers F.Cu F.Paste F.Mask) (roundrect_rratio 0.25) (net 7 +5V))
  (pad 6 smd roundrect (at -5.6625 -1.25 270) (size 1.475 0.3) (layers F.Cu F.Paste F.Mask) (roundrect_rratio 0.25) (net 2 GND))
  (pad 5 smd roundrect (at -5.6625 -1.75 270) (size 1.475 0.3) (layers F.Cu F.Paste F.Mask) (roundrect_rratio 0.25))
  (pad 4 smd roundrect (at -5.6625 -2.25 270) (size 1.475 0.3) (layers F.Cu F.Paste F.Mask) (roundrect_rratio 0.25))
  (pad 3 smd roundrect (at -5.6625 -2.75 270) (size 1.475 0.3) (layers F.Cu F.Paste F.Mask) (roundrect_rratio 0.25))
  (pad 2 smd roundrect (at -5.6625 -3.25 270) (size 1.475 0.3) (layers F.Cu F.Paste F.Mask) (roundrect_rratio 0.25))
  (pad 1 smd roundrect (at -5.6625 -3.75 270) (size 1.475 0.3) (layers F.Cu F.Paste F.Mask) (roundrect_rratio 0.25)))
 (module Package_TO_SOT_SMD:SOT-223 (layer F.Cu) (at 135.63 60.09)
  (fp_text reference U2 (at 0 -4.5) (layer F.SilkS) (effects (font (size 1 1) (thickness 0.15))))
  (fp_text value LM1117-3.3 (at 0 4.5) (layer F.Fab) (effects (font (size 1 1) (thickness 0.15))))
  (pad 1 smd rect (at -3.15 -2.3) (size 2 1.5) (layers F.Cu F.Paste F.Mask) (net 2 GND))
  (pad 3 smd rect (at -3.15 2.3) (size 2 1.5) (layers F.Cu F.Paste F.Mask) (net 7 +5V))
  (pad 2 smd rect (at -3.15 0) (size 2 1.5) (layers F.Cu F.Paste F.Mask) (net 32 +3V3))
  (pad 4 smd rect (at 3.15 0) (size 2 3.8) (layers F.Cu F.Paste F.Mask) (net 32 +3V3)))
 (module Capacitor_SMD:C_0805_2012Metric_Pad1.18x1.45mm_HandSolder (layer F.Cu) (at 141.01 85.0425 270)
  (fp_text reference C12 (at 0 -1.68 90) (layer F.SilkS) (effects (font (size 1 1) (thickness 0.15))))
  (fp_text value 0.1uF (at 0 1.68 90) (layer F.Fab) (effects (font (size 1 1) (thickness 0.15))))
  (pad 2 smd roundrect (at 1.0375 0 270) (size 1.175 1.45) (layers F.Cu F.Paste F.Mask) (roundrect_rratio 0.2127659574468085) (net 2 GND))
  (pad 1 smd roundrect (at -1.0375 0 270) (size 1.175 1.45) (layers F.Cu F.Paste F.Mask) (roundrect_rratio 0.2127659574468085) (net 7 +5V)))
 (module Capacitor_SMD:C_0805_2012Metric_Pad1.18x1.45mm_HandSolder (layer F.Cu) (at 143.11 60.69)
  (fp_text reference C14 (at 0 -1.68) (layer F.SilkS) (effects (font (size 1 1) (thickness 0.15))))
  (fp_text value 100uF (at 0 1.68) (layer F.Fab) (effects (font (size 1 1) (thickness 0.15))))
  (pad 2 smd roundrect (at 1.0375 0) (size 1.175 1.45) (layers F.Cu F.Paste F.Mask) (roundrect_rratio 0.2127659574468085) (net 2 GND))
  (pad 1 smd roundrect (at -1.0375 0) (size 1.175 1.45) (layers F.Cu F.Paste F.Mask) (roundrect_rratio 0.2127659574468085) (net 32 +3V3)))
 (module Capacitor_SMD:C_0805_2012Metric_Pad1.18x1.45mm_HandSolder (layer F.Cu) (at 148.41 52.9925 270)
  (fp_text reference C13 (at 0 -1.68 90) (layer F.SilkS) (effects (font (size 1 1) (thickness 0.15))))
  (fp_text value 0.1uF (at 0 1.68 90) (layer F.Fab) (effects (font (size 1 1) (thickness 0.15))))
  (pad 2 smd roundrect (at 1.0375 0 270) (size 1.175 1.45) (layers F.Cu F.Paste F.Mask) (roundrect_rratio 0.2127659574468085) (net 2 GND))
  (pad 1 smd roundrect (at -1.0375 0 270) (size 1.175 1.45) (layers F.Cu F.Paste F.Mask) (roundrect_rratio 0.2127659574468085) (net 7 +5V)))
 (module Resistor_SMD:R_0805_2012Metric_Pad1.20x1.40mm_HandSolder (layer F.Cu) (at 113.11 81.43 270)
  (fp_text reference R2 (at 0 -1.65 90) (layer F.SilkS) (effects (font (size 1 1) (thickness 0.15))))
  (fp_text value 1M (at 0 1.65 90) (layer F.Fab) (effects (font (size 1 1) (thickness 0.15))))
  (pad 1 smd roundrect (at -1 0 270) (size 1.2 1.4) (layers F.Cu F.Paste F.Mask) (roundrect_rratio 0.2083325) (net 26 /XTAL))
  (pad 2 smd roundrect (at 1 0 270) (size 1.2 1.4) (layers F.Cu F.Paste F.Mask) (roundrect_rratio 0.2083325) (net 27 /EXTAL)))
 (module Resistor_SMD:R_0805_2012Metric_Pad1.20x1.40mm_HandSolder (layer F.Cu) (at 141.76 71.48 180)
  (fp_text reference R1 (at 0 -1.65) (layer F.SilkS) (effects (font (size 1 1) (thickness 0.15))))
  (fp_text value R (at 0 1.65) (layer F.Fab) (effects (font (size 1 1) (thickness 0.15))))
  (pad 2 smd roundrect (at 1 0 180) (size 1.2 1.4) (layers F.Cu F.Paste F.Mask) (roundrect_rratio 0.2083325) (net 38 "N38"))
  (pad 1 smd roundrect (at -1 0 180) (size 1.2 1.4) (layers F.Cu F.Paste F.Mask) (roundrect_rratio 0.2083325) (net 4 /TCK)))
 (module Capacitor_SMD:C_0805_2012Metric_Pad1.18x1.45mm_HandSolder (layer F.Cu) (at 113.17 77.2725 90)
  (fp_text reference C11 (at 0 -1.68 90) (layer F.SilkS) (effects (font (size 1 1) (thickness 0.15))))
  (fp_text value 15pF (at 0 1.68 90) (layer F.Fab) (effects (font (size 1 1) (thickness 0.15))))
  (pad 1 smd roundrect (at -1.0375 0 90) (size 1.175 1.45) (layers F.Cu F.Paste F.Mask) (roundrect_rratio 0.2127659574468085) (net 26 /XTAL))
  (pad 2 smd roundrect (at 1.0375 0 90) (size 1.175 1.45) (layers F.Cu F.Paste F.Mask) (roundrect_rratio 0.2127659574468085) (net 2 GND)))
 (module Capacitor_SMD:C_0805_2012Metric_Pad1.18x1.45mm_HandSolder (layer F.Cu) (at 113.14 85.69 270)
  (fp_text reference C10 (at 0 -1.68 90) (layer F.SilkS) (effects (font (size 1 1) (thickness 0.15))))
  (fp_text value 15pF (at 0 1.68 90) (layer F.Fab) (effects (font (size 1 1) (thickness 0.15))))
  (pad 1 smd roundrect (at -1.0375 0 270) (size 1.175 1.45) (layers F.Cu F.Paste F.Mask) (roundrect_rratio 0.2127659574468085)
   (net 27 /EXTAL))
  (pad 2 smd roundrect (at 1.0375 0 270) (size 1.175 1.45) (layers F.Cu F.Paste F.Mask) (roundrect_rratio 0.2127659574468085) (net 2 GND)))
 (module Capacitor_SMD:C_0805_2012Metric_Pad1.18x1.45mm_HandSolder (layer F.Cu) (at 132.89 53.25 270)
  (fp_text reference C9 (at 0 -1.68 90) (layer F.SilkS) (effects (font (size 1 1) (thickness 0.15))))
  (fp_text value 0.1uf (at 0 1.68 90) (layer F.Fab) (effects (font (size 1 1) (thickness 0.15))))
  (pad 2 smd roundrect (at 1.0375 0 270) (size 1.175 1.45) (layers F.Cu F.Paste F.Mask) (roundrect_rratio 0.2127659574468085) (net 2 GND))
  (pad 1 smd roundrect (at -1.0375 0 270) (size 1.175 1.45) (layers F.Cu F.Paste F.Mask) (roundrect_rratio 0.2127659574468085) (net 7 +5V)))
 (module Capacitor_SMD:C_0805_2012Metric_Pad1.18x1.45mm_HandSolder (layer F.Cu) (at 136.52 53.2325 270)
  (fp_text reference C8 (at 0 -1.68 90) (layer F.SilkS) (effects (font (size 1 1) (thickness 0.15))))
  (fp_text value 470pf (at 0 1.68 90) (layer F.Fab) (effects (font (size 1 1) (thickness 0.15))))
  (pad 2 smd roundrect (at 1.0375 0 270) (size 1.175 1.45) (layers F.Cu F.Paste F.Mask) (roundrect_rratio 0.2127659574468085) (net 2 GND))
  (pad 1 smd roundrect (at -1.0375 0 270) (size 1.175 1.45) (layers F.Cu F.Paste F.Mask) (roundrect_rratio 0.2127659574468085) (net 7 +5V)))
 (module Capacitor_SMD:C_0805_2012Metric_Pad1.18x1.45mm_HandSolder (layer F.Cu) (at 126.455 68.8325 90)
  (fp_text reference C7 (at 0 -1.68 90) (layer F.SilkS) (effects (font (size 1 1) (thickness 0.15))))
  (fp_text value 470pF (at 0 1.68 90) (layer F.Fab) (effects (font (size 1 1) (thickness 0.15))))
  (pad 2 smd roundrect (at 1.0375 0 90) (size 1.175 1.45) (layers F.Cu F.Paste F.Mask) (roundrect_rratio 0.2127659574468085) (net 2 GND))
  (pad 1 smd roundrect (at -1.0375 0 90) (size 1.175 1.45) (layers F.Cu F.Paste F.Mask) (roundrect_rratio 0.2127659574468085)
   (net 39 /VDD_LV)))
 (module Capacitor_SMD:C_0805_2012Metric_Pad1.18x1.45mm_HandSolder (layer F.Cu) (at 128.79 53.2325 270)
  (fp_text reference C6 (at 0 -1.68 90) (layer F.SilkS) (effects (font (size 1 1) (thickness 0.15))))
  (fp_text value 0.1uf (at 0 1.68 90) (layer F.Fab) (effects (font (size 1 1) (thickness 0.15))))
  (pad 2 smd roundrect (at 1.0375 0 270) (size 1.175 1.45) (layers F.Cu F.Paste F.Mask) (roundrect_rratio 0.2127659574468085) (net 2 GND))
  (pad 1 smd roundrect (at -1.0375 0 270) (size 1.175 1.45) (layers F.Cu F.Paste F.Mask) (roundrect_rratio 0.2127659574468085) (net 7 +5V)))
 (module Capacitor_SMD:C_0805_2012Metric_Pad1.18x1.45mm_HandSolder (layer F.Cu) (at 130.265 68.8325 90)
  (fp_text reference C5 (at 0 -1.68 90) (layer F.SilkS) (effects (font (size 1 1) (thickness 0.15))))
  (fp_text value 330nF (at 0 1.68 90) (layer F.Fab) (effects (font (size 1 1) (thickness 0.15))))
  (pad 2 smd roundrect (at 1.0375 0 90) (size 1.175 1.45) (layers F.Cu F.Paste F.Mask) (roundrect_rratio 0.2127659574468085) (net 2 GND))
  (pad 1 smd roundrect (at -1.0375 0 90) (size 1.175 1.45) (layers F.Cu F.Paste F.Mask) (roundrect_rratio 0.2127659574468085)
   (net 39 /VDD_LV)))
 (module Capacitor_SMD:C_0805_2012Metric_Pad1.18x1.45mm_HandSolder (layer F.Cu) (at 139.84 53.1725 270)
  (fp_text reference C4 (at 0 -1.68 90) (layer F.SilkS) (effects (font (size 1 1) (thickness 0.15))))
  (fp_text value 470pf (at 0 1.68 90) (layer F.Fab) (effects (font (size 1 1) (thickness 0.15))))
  (pad 2 smd roundrect (at 1.0375 0 270) (size 1.175 1.45) (layers F.Cu F.Paste F.Mask) (roundrect_rratio 0.2127659574468085) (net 2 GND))
  (pad 1 smd roundrect (at -1.0375 0 270) (size 1.175 1.45) (layers F.Cu F.Paste F.Mask) (roundrect_rratio 0.2127659574468085) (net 7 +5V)))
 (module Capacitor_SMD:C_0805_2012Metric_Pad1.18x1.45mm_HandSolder (layer F.Cu) (at 134.075 68.8325 90)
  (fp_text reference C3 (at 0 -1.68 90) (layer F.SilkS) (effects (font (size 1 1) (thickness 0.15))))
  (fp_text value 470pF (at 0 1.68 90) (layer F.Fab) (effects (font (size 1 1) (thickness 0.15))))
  (pad 2 smd roundrect (at 1.0375 0 90) (size 1.175 1.45) (layers F.Cu F.Paste F.Mask) (roundrect_rratio 0.2127659574468085) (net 2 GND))
  (pad 1 smd roundrect (at -1.0375 0 90) (size 1.175 1.45) (layers F.Cu F.Paste F.Mask) (roundrect_rratio 0.2127659574468085)
   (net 39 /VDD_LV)))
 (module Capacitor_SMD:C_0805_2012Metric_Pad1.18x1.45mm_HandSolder (layer F.Cu) (at 145.33 52.9725 270)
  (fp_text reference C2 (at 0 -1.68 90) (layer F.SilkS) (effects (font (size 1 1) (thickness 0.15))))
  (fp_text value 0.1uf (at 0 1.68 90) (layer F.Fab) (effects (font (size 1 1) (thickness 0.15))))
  (pad 2 smd roundrect (at 1.0375 0 270) (size 1.175 1.45) (layers F.Cu F.Paste F.Mask) (roundrect_rratio 0.2127659574468085) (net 2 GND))
  (pad 1 smd roundrect (at -1.0375 0 270) (size 1.175 1.45) (layers F.Cu F.Paste F.Mask) (roundrect_rratio 0.2127659574468085) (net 7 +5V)))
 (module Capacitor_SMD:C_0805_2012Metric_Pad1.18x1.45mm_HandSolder (layer F.Cu) (at 142.51 53.0775 270)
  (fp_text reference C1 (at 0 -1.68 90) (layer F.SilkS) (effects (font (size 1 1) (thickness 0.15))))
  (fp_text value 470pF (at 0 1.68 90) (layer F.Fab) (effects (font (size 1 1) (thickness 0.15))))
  (pad 2 smd roundrect (at 1.0375 0 270) (size 1.175 1.45) (layers F.Cu F.Paste F.Mask) (roundrect_rratio 0.2127659574468085) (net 2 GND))
  (pad 1 smd roundrect (at -1.0375 0 270) (size 1.175 1.45) (layers F.Cu F.Paste F.Mask) (roundrect_rratio 0.2127659574468085) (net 7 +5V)))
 (gr_circle (center 102.97 73.178815) (end 104.01 73.738815) (layer Edge.Cuts) (width 0.1))
 (segment (start 145.2825 52.2725) (end 145.05 52.04) (width 0.25) (layer F.Cu) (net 7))
 (segment (start 106.68 73.66) (end 105.41 72.39) (width 0.25) (layer VCC) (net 7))
 (segment (start 121.92 73.66) (end 106.68 73.66) (width 0.25) (layer VCC) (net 7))
 (segment (start 109.22 99.06) (end 109.22 91.44) (width 0.25) (layer VCC) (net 7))
 (segment (start 105.41 87.63) (end 105.41 72.39) (width 0.25) (layer VCC) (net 7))
 (segment (start 109.22 91.44) (end 105.41 87.63) (width 0.25) (layer VCC) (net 7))
 (segment (start 145.2825 54.3475) (end 145.05 54.115) (width 0.25) (layer F.Cu) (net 2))
 (segment (start 117.588998 72.39) (end 118.11 72.39) (width 0.25) (layer GND) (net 7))
 (segment (start 113.665 68.466002) (end 117.588998 72.39) (width 0.25) (layer GND) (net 7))
 (segment (start 113.665 66.04) (end 113.665 68.466002) (width 0.25) (layer GND) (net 7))
 (segment (start 118.745 66.04) (end 130.175 54.61) (width 0.25) (layer GND) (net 7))
 (segment (start 113.665 66.04) (end 118.745 66.04) (width 0.25) (layer GND) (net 7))
 (segment (start 130.175 64.135) (end 147.32 81.28) (width 0.25) (layer GND) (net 7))
 (segment (start 130.175 54.61) (end 130.175 64.135) (width 0.25) (layer GND) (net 7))
 (segment (start 147.32 92.075) (end 141.605 97.79) (width 0.25) (layer GND) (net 7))
 (segment (start 147.32 81.28) (end 147.32 92.075) (width 0.25) (layer GND) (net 7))
 (segment (start 118.11 73.66) (end 125.73 81.28) (width 0.25) (layer GND) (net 7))
 (segment (start 118.11 72.39) (end 118.11 73.66) (width 0.25) (layer GND) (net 7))
 (segment (start 147.55 79.33) (end 147.75 79.33) (width 0.25) (layer F.Cu) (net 5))
 (segment (start 103.695001 70.929999) (end 106.68 67.945) (width 0.25) (layer VCC) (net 32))
 (segment (start 103.695001 84.899999) (end 103.695001 70.929999) (width 0.25) (layer VCC) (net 32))
 (segment (start 102.87 85.725) (end 103.695001 84.899999) (width 0.25) (layer VCC) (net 32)))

